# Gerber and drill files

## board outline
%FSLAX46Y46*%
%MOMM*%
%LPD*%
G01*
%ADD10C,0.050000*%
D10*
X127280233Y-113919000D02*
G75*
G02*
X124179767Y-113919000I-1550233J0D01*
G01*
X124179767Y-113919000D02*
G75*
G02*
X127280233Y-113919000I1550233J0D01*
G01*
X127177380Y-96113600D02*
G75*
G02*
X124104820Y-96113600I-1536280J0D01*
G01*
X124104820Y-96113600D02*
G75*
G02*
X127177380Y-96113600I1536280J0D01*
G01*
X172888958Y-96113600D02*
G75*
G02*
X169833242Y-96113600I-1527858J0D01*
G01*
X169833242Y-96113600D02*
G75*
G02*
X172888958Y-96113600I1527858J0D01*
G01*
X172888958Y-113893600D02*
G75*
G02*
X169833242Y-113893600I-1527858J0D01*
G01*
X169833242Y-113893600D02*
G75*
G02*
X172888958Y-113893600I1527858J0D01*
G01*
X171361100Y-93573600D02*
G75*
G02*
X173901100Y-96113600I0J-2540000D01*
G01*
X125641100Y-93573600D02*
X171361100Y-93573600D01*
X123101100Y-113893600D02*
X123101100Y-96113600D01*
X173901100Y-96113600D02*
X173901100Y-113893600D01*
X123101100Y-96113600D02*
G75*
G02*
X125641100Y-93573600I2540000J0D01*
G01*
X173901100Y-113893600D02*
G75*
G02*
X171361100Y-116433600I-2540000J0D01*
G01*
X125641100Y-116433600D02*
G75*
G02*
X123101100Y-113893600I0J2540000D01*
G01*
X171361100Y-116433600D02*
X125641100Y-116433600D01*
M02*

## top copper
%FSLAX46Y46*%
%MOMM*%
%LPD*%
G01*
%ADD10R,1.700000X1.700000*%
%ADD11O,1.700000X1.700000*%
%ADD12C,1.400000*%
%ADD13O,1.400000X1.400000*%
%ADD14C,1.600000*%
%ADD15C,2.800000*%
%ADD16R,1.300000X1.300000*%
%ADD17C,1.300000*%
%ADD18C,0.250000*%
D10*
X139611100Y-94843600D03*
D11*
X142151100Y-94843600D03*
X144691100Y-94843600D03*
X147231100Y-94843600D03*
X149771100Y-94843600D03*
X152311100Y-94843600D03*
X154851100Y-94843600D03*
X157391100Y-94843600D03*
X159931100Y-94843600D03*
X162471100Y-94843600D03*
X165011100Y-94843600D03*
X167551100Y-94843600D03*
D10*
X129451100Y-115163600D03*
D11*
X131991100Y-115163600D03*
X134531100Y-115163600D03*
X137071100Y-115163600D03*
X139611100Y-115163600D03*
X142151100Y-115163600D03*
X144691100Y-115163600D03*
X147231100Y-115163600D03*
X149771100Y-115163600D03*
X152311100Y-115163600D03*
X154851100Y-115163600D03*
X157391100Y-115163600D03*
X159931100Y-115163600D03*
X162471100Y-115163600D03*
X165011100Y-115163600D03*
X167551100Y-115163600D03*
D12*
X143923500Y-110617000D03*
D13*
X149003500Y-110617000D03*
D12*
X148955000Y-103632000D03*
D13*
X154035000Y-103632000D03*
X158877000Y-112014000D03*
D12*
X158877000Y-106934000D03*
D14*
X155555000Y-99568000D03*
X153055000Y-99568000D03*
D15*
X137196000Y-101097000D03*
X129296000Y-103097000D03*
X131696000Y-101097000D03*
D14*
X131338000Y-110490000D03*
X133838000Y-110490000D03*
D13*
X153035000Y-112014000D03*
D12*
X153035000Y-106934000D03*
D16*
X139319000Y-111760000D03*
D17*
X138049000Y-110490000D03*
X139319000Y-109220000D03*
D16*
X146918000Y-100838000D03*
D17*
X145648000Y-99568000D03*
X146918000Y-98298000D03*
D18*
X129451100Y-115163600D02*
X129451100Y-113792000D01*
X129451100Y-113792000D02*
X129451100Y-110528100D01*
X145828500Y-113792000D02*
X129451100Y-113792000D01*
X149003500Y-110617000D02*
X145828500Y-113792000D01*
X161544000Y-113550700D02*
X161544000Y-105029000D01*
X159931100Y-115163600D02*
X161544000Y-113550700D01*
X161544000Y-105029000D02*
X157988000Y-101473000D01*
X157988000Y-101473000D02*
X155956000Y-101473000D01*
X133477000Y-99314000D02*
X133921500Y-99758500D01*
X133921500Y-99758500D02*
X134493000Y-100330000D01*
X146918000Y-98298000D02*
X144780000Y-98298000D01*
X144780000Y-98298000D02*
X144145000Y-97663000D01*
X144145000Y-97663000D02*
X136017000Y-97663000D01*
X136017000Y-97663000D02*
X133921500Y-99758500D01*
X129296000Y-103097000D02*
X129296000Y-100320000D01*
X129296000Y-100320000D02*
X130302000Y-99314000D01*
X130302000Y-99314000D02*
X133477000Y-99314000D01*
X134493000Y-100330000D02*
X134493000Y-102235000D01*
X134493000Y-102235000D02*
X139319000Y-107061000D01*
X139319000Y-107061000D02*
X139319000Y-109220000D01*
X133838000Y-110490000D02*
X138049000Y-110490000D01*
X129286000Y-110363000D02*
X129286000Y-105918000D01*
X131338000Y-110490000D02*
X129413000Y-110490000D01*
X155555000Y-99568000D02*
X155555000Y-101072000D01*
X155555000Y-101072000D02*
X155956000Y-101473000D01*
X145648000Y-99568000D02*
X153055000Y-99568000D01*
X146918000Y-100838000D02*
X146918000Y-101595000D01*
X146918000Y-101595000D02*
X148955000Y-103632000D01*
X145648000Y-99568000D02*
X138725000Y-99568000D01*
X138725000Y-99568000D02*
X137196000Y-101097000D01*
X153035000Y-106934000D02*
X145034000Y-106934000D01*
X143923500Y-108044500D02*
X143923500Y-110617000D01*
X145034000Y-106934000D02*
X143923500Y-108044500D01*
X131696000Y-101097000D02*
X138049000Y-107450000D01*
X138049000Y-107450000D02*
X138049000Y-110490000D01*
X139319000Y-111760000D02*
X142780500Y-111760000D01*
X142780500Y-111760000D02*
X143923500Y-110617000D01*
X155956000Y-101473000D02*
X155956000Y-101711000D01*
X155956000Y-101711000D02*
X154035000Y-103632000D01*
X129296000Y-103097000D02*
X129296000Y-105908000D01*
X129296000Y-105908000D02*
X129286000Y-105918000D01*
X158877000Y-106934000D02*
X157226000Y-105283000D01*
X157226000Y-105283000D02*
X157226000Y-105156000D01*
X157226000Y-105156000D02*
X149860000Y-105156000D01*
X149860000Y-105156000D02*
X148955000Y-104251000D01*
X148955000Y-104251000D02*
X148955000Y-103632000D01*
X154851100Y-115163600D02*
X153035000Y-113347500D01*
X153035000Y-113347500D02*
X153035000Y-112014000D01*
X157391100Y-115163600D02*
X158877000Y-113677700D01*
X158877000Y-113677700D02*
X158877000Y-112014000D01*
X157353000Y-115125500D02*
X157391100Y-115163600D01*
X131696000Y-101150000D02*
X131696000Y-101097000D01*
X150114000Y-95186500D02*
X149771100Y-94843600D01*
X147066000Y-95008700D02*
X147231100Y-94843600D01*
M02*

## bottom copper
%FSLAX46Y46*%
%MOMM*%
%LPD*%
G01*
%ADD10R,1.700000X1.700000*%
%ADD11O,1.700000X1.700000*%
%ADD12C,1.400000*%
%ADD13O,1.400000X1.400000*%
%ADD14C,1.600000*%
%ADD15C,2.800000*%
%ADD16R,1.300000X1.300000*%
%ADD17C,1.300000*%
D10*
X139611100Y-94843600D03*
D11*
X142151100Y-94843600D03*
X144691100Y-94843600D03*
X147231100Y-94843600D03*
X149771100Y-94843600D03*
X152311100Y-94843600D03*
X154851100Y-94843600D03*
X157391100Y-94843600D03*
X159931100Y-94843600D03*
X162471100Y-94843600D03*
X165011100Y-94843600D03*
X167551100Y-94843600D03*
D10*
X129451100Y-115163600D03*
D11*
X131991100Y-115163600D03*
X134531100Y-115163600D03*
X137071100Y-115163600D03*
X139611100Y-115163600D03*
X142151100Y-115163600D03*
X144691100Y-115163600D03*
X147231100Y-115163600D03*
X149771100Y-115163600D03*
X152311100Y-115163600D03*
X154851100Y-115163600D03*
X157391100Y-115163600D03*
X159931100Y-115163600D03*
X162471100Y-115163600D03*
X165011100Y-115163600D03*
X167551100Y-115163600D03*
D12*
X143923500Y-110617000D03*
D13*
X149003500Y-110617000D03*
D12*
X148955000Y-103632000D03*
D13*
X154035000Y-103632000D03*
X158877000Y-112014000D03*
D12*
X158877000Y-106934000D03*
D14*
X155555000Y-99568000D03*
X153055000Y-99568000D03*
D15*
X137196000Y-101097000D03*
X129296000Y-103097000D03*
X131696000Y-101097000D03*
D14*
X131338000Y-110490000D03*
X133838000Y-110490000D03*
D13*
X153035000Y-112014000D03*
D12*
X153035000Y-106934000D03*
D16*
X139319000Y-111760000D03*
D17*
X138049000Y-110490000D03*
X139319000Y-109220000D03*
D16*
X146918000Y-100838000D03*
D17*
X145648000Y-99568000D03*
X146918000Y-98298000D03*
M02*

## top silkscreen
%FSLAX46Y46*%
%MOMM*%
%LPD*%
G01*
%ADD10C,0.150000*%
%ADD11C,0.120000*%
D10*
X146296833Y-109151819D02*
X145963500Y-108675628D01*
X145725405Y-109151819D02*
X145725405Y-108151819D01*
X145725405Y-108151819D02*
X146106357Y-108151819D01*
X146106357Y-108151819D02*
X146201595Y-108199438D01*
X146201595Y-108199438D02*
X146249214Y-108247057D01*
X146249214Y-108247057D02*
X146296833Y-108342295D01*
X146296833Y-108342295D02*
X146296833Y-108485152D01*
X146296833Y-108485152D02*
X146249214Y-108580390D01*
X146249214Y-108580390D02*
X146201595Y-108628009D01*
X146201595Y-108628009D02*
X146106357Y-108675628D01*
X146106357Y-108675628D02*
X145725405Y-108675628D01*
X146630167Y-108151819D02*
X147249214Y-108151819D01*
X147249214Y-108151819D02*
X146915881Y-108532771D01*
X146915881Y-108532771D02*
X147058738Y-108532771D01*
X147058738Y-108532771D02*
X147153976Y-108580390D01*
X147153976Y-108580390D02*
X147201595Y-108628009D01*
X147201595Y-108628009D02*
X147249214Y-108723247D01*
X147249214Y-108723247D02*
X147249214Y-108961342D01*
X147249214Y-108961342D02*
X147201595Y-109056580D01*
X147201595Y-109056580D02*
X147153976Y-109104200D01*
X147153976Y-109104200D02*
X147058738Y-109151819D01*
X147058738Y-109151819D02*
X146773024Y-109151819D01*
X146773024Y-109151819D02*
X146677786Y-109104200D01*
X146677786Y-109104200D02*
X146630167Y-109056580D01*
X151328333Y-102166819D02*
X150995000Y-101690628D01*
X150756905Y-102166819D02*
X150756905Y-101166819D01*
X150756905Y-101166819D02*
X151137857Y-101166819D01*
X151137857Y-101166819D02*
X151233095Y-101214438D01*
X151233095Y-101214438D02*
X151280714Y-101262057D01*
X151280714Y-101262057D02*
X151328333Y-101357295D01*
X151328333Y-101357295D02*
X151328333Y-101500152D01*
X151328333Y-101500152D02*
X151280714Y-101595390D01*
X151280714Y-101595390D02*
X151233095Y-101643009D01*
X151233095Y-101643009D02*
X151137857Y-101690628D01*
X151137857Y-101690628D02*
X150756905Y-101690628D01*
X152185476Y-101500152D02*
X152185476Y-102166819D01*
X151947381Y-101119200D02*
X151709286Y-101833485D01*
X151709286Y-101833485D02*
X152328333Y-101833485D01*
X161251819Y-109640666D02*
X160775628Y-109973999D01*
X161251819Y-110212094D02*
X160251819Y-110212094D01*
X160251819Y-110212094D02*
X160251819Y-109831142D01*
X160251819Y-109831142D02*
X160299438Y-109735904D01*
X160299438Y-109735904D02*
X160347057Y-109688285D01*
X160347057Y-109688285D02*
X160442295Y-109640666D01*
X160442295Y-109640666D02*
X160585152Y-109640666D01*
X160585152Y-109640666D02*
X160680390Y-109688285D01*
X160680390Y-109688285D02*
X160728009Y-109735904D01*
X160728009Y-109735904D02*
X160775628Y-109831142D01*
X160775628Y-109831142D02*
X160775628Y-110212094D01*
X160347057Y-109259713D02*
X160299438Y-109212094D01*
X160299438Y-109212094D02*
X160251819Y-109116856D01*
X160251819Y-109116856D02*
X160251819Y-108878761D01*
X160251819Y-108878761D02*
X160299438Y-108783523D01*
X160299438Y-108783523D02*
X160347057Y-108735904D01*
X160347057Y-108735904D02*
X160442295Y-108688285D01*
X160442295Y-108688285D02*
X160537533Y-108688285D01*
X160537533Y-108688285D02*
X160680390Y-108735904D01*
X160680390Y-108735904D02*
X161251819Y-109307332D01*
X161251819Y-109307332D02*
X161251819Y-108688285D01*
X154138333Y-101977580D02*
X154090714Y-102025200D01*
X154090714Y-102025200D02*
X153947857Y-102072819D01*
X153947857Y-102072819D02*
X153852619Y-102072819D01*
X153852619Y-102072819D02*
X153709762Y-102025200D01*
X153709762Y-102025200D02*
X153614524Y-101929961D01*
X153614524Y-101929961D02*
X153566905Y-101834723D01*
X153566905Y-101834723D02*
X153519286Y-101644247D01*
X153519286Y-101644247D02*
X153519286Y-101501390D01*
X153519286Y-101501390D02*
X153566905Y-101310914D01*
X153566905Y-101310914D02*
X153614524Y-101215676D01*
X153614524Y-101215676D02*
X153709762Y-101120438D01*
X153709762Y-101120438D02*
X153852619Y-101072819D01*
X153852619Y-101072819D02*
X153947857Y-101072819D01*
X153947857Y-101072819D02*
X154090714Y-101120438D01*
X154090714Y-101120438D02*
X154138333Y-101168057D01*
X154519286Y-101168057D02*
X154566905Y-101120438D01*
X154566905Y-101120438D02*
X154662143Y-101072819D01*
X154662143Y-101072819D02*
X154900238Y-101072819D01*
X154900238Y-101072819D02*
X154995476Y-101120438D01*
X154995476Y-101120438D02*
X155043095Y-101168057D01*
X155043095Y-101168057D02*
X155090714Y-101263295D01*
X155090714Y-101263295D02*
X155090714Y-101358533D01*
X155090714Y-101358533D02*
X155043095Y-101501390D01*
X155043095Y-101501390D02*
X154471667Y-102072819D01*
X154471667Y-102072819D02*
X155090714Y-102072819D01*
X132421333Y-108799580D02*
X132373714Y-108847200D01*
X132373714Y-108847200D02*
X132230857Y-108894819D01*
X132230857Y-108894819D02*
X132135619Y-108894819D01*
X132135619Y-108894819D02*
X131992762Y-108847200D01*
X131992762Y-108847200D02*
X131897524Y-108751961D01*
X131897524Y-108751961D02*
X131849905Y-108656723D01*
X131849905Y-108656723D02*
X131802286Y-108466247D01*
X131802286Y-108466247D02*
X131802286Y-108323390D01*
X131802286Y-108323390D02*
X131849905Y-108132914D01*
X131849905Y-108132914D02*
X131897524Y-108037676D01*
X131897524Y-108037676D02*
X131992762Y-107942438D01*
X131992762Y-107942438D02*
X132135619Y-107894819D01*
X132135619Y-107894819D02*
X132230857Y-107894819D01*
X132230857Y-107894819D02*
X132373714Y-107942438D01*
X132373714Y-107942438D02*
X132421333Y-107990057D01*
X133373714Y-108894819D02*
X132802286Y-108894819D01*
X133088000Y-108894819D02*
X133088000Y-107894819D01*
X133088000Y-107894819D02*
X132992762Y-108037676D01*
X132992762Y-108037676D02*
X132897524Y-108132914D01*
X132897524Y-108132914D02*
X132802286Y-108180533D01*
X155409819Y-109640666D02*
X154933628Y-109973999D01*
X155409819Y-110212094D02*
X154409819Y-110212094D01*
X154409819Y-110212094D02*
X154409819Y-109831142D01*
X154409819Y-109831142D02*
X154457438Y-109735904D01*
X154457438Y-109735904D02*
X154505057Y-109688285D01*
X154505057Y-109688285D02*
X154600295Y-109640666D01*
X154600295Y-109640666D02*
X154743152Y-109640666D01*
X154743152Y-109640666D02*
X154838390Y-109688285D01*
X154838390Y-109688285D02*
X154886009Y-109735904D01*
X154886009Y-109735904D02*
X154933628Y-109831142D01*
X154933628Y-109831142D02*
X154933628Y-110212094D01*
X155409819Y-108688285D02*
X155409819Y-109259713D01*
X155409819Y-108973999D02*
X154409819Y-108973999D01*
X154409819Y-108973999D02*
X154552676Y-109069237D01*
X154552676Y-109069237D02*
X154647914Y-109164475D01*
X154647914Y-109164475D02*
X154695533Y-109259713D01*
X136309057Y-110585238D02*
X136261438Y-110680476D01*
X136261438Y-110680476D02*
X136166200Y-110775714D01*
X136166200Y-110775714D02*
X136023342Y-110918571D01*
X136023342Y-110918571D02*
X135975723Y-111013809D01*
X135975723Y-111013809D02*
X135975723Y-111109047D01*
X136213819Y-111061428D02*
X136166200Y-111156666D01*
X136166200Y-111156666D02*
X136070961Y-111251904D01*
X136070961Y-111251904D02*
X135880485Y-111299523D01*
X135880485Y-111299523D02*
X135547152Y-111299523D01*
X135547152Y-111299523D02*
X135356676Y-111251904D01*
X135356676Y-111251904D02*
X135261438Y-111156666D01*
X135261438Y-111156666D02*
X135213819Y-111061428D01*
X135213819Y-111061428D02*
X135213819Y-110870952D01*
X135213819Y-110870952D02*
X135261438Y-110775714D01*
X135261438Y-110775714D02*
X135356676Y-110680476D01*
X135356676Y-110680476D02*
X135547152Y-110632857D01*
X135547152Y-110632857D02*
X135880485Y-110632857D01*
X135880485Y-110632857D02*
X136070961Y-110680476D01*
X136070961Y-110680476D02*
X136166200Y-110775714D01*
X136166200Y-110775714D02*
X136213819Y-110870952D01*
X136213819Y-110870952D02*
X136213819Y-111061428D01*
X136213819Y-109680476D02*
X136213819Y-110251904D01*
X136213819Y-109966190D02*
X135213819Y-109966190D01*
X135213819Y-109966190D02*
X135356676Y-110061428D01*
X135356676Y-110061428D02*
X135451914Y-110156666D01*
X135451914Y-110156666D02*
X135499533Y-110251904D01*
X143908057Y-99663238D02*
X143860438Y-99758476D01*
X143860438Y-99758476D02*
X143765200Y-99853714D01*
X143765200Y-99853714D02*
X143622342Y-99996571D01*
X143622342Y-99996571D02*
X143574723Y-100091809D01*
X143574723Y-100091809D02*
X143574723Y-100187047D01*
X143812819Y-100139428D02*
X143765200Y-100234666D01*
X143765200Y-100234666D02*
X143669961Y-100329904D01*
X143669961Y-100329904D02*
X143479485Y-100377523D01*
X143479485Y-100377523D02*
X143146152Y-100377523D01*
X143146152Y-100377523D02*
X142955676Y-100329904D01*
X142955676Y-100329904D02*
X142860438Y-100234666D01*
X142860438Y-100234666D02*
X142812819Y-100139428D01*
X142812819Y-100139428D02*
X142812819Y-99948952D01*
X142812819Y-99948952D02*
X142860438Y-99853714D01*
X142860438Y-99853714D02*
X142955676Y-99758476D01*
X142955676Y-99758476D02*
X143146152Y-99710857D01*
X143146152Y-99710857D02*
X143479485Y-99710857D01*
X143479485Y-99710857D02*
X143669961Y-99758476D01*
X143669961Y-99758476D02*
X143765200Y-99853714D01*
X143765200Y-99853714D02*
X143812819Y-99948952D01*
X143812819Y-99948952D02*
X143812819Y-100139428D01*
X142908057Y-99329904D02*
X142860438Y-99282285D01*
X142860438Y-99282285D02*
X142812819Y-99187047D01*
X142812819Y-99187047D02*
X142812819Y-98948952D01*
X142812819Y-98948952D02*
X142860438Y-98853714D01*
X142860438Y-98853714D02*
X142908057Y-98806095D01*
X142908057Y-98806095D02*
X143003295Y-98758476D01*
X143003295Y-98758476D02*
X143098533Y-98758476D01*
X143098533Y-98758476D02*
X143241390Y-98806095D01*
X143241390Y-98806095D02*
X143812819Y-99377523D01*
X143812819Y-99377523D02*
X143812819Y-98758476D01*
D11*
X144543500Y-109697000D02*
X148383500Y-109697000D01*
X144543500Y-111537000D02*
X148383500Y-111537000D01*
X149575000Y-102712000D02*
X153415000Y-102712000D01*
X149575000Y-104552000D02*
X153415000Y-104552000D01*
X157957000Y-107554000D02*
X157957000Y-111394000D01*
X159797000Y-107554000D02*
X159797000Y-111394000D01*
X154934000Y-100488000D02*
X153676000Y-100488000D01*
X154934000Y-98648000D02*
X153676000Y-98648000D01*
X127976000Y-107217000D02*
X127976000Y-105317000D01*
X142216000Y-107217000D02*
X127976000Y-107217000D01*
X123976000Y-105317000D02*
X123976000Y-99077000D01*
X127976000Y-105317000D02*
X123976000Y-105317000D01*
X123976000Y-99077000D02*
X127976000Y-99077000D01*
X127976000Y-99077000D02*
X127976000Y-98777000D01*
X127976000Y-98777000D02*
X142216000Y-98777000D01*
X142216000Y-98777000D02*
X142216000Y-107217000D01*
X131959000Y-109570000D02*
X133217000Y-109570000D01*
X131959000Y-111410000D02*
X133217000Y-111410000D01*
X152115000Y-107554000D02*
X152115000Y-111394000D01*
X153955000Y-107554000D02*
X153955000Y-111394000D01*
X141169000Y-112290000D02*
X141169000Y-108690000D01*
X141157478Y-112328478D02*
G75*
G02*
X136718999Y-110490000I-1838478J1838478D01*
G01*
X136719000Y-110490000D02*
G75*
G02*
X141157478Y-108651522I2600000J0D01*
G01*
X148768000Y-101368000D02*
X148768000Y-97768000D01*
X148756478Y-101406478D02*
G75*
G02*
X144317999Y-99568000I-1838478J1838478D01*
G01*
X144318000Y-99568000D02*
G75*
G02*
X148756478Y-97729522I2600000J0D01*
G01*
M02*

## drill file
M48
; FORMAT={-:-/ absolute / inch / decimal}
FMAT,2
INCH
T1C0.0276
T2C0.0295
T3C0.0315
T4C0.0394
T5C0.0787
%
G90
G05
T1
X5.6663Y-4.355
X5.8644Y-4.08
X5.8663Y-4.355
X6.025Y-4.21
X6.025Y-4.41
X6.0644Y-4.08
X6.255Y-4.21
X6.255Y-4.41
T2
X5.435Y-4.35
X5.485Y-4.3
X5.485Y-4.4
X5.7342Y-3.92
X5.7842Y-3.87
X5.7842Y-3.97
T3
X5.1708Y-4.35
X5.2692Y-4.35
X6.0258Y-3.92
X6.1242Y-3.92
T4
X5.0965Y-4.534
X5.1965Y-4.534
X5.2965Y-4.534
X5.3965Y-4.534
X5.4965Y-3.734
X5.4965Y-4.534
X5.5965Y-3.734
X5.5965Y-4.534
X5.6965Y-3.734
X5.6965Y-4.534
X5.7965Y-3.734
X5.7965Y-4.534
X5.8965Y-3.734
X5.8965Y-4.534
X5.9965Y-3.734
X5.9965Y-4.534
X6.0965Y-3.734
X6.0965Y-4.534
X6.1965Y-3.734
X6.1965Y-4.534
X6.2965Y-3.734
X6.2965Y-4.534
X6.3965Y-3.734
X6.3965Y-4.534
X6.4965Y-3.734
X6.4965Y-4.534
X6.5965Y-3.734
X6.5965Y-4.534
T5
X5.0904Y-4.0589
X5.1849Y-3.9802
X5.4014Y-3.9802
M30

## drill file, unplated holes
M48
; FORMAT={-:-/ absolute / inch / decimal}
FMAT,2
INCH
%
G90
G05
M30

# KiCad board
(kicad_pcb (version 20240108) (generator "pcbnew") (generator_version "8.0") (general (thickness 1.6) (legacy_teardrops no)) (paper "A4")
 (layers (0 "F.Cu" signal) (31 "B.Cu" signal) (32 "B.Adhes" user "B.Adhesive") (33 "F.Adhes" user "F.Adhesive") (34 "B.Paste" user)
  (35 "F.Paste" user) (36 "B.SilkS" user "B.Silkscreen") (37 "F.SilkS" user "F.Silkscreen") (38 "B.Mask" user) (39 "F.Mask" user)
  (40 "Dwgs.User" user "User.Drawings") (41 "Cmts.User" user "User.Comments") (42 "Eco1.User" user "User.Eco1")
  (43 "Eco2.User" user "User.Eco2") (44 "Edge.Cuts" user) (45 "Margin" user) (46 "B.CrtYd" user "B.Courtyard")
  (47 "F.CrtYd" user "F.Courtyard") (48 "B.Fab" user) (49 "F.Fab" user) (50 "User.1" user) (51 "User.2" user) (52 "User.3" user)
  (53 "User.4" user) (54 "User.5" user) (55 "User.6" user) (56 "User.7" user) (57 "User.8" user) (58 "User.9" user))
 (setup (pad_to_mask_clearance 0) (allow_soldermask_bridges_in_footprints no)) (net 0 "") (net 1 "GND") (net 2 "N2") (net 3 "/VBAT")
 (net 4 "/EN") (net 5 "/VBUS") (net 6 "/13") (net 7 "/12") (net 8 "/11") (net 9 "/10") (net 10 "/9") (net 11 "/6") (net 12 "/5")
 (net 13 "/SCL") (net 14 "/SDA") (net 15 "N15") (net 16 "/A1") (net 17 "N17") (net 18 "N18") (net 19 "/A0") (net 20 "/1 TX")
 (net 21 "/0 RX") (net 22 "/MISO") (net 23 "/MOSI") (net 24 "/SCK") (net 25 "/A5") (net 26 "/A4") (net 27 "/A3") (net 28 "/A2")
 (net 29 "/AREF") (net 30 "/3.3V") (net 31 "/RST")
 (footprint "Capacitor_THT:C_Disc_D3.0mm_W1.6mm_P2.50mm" (layer "F.Cu") (at 155.555 99.568 180)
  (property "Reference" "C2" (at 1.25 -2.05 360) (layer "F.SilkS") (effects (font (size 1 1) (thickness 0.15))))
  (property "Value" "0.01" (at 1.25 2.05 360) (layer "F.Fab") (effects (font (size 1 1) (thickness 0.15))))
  (fp_line (start 0.621 0.92) (end 1.879 0.92) (stroke (width 0.12) (type solid)) (layer "F.SilkS"))
  (fp_line (start 0.621 -0.92) (end 1.879 -0.92) (stroke (width 0.12) (type solid)) (layer "F.SilkS"))
  (pad "1" thru_hole circle (at 0 0 180) (size 1.6 1.6) (drill 0.8) (layers "*.Cu" "*.Mask") (remove_unused_layers no) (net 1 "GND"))
  (pad "2" thru_hole circle (at 2.5 0 180) (size 1.6 1.6) (drill 0.8) (layers "*.Cu" "*.Mask") (remove_unused_layers no) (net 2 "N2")))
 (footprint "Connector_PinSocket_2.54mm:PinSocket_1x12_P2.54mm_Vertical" (layer "F.Cu") (at 139.6111 94.8436 90)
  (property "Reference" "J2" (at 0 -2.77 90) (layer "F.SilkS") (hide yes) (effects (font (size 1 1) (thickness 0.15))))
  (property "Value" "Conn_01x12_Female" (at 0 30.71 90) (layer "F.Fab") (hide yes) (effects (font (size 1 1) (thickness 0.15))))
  (pad "1" thru_hole rect (at 0 0 90) (size 1.7 1.7) (drill 1) (layers "*.Cu" "*.Mask") (remove_unused_layers no) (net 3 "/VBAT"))
  (pad "2" thru_hole oval (at 0 2.54 90) (size 1.7 1.7) (drill 1) (layers "*.Cu" "*.Mask") (remove_unused_layers no) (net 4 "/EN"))
  (pad "3" thru_hole oval (at 0 5.08 90) (size 1.7 1.7) (drill 1) (layers "*.Cu" "*.Mask") (remove_unused_layers no) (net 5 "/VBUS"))
  (pad "4" thru_hole oval (at 0 7.62 90) (size 1.7 1.7) (drill 1) (layers "*.Cu" "*.Mask") (remove_unused_layers no) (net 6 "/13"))
  (pad "5" thru_hole oval (at 0 10.16 90) (size 1.7 1.7) (drill 1) (layers "*.Cu" "*.Mask") (remove_unused_layers no) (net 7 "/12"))
  (pad "6" thru_hole oval (at 0 12.7 90) (size 1.7 1.7) (drill 1) (layers "*.Cu" "*.Mask") (remove_unused_layers no) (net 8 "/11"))
  (pad "7" thru_hole oval (at 0 15.24 90) (size 1.7 1.7) (drill 1) (layers "*.Cu" "*.Mask") (remove_unused_layers no) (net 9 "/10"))
  (pad "8" thru_hole oval (at 0 17.78 90) (size 1.7 1.7) (drill 1) (layers "*.Cu" "*.Mask") (remove_unused_layers no) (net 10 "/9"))
  (pad "9" thru_hole oval (at 0 20.32 90) (size 1.7 1.7) (drill 1) (layers "*.Cu" "*.Mask") (remove_unused_layers no) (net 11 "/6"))
  (pad "10" thru_hole oval (at 0 22.86 90) (size 1.7 1.7) (drill 1) (layers "*.Cu" "*.Mask") (remove_unused_layers no) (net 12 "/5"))
  (pad "11" thru_hole oval (at 0 25.4 90) (size 1.7 1.7) (drill 1) (layers "*.Cu" "*.Mask") (remove_unused_layers no) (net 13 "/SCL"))
  (pad "12" thru_hole oval (at 0 27.94 90) (size 1.7 1.7) (drill 1) (layers "*.Cu" "*.Mask") (remove_unused_layers no) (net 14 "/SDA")))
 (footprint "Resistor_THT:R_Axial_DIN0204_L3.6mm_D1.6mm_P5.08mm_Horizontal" (layer "F.Cu") (at 153.035 106.934 -90)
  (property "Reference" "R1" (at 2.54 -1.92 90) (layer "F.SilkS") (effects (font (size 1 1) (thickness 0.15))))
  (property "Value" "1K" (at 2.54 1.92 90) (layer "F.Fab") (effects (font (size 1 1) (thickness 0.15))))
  (fp_line (start 0.62 0.92) (end 4.46 0.92) (stroke (width 0.12) (type solid)) (layer "F.SilkS"))
  (fp_line (start 0.62 -0.92) (end 4.46 -0.92) (stroke (width 0.12) (type solid)) (layer "F.SilkS"))
  (pad "1" thru_hole circle (at 0 0 270) (size 1.4 1.4) (drill 0.7) (layers "*.Cu" "*.Mask") (remove_unused_layers no) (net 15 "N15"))
  (pad "2" thru_hole oval (at 5.08 0 270) (size 1.4 1.4) (drill 0.7) (layers "*.Cu" "*.Mask") (remove_unused_layers no) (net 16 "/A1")))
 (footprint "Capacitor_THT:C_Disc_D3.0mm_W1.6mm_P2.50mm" (layer "F.Cu") (at 131.338 110.49)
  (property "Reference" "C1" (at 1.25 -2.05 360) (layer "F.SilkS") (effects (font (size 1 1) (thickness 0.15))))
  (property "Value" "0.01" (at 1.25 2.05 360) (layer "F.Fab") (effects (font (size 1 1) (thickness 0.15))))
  (fp_line (start 0.621 -0.92) (end 1.879 -0.92) (stroke (width 0.12) (type solid)) (layer "F.SilkS"))
  (fp_line (start 0.621 0.92) (end 1.879 0.92) (stroke (width 0.12) (type solid)) (layer "F.SilkS"))
  (pad "1" thru_hole circle (at 0 0) (size 1.6 1.6) (drill 0.8) (layers "*.Cu" "*.Mask") (remove_unused_layers no) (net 1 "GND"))
  (pad "2" thru_hole circle (at 2.5 0) (size 1.6 1.6) (drill 0.8) (layers "*.Cu" "*.Mask") (remove_unused_layers no) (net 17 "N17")))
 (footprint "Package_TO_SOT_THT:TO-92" (layer "F.Cu") (at 146.918 100.838 90)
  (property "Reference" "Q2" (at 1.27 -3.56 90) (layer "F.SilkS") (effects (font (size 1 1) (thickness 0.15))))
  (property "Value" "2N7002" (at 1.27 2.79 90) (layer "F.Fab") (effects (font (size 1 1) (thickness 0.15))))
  (fp_line (start -0.53 1.85) (end 3.07 1.85) (stroke (width 0.12) (type solid)) (layer "F.SilkS"))
  (fp_arc (start 1.27 -2.6) (mid 3.672087 -0.994977) (end 3.108478 1.838478) (stroke (width 0.12) (type solid)) (layer "F.SilkS"))
  (fp_arc (start -0.568478 1.838478) (mid -1.132087 -0.994977) (end 1.27 -2.6) (stroke (width 0.12) (type solid)) (layer "F.SilkS"))
  (pad "1" thru_hole rect (at 0 0 90) (size 1.3 1.3) (drill 0.75) (layers "*.Cu" "*.Mask") (remove_unused_layers no) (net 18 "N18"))
  (pad "2" thru_hole circle (at 1.27 -1.27 90) (size 1.3 1.3) (drill 0.75) (layers "*.Cu" "*.Mask") (remove_unused_layers no) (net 2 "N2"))
  (pad "3" thru_hole circle (at 2.54 0 90) (size 1.3 1.3) (drill 0.75) (layers "*.Cu" "*.Mask") (remove_unused_layers no) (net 1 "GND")))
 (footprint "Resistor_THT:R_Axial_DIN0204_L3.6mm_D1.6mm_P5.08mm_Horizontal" (layer "F.Cu") (at 158.877 106.934 -90)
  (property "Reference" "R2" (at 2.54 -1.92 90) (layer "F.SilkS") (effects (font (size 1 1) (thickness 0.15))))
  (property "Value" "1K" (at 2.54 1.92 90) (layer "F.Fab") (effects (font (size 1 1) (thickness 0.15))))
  (fp_line (start 0.62 0.92) (end 4.46 0.92) (stroke (width 0.12) (type solid)) (layer "F.SilkS"))
  (fp_line (start 0.62 -0.92) (end 4.46 -0.92) (stroke (width 0.12) (type solid)) (layer "F.SilkS"))
  (pad "1" thru_hole circle (at 0 0 270) (size 1.4 1.4) (drill 0.7) (layers "*.Cu" "*.Mask") (remove_unused_layers no) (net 18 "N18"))
  (pad "2" thru_hole oval (at 5.08 0 270) (size 1.4 1.4) (drill 0.7) (layers "*.Cu" "*.Mask") (remove_unused_layers no) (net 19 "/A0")))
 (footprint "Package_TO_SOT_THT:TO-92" (layer "F.Cu") (at 139.319 111.76 90)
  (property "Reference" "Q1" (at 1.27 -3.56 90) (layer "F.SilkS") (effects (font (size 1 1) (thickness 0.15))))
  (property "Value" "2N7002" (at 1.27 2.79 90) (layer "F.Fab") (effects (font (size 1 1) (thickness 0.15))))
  (fp_line (start -0.53 1.85) (end 3.07 1.85) (stroke (width 0.12) (type solid)) (layer "F.SilkS"))
  (fp_arc (start 1.27 -2.6) (mid 3.672087 -0.994977) (end 3.108478 1.838478) (stroke (width 0.12) (type solid)) (layer "F.SilkS"))
  (fp_arc (start -0.568478 1.838478) (mid -1.132087 -0.994977) (end 1.27 -2.6) (stroke (width 0.12) (type solid)) (layer "F.SilkS"))
  (pad "1" thru_hole rect (at 0 0 90) (size 1.3 1.3) (drill 0.75) (layers "*.Cu" "*.Mask") (remove_unused_layers no) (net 15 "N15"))
  (pad "2" thru_hole circle (at 1.27 -1.27 90) (size 1.3 1.3) (drill 0.75) (layers "*.Cu" "*.Mask") (remove_unused_layers no) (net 17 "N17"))
  (pad "3" thru_hole circle (at 2.54 0 90) (size 1.3 1.3) (drill 0.75) (layers "*.Cu" "*.Mask") (remove_unused_layers no) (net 1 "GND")))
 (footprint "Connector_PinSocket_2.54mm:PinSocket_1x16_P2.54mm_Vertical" (layer "F.Cu") (at 129.4511 115.1636 90)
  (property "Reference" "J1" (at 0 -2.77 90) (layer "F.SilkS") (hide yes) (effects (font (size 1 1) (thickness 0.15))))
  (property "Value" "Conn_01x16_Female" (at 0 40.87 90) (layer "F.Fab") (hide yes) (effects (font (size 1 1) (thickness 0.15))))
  (pad "1" thru_hole rect (at 0 0 90) (size 1.7 1.7) (drill 1) (layers "*.Cu" "*.Mask") (remove_unused_layers no) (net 1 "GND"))
  (pad "2" thru_hole oval (at 0 2.54 90) (size 1.7 1.7) (drill 1) (layers "*.Cu" "*.Mask") (remove_unused_layers no) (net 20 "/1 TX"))
  (pad "3" thru_hole oval (at 0 5.08 90) (size 1.7 1.7) (drill 1) (layers "*.Cu" "*.Mask") (remove_unused_layers no) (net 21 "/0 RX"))
  (pad "4" thru_hole oval (at 0 7.62 90) (size 1.7 1.7) (drill 1) (layers "*.Cu" "*.Mask") (remove_unused_layers no) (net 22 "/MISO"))
  (pad "5" thru_hole oval (at 0 10.16 90) (size 1.7 1.7) (drill 1) (layers "*.Cu" "*.Mask") (remove_unused_layers no) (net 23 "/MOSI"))
  (pad "6" thru_hole oval (at 0 12.7 90) (size 1.7 1.7) (drill 1) (layers "*.Cu" "*.Mask") (remove_unused_layers no) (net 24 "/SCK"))
  (pad "7" thru_hole oval (at 0 15.24 90) (size 1.7 1.7) (drill 1) (layers "*.Cu" "*.Mask") (remove_unused_layers no) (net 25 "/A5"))
  (pad "8" thru_hole oval (at 0 17.78 90) (size 1.7 1.7) (drill 1) (layers "*.Cu" "*.Mask") (remove_unused_layers no) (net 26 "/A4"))
  (pad "9" thru_hole oval (at 0 20.32 90) (size 1.7 1.7) (drill 1) (layers "*.Cu" "*.Mask") (remove_unused_layers no) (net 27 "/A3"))
  (pad "10" thru_hole oval (at 0 22.86 90) (size 1.7 1.7) (drill 1) (layers "*.Cu" "*.Mask") (remove_unused_layers no) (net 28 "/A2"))
  (pad "11" thru_hole oval (at 0 25.4 90) (size 1.7 1.7) (drill 1) (layers "*.Cu" "*.Mask") (remove_unused_layers no) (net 16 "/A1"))
  (pad "12" thru_hole oval (at 0 27.94 90) (size 1.7 1.7) (drill 1) (layers "*.Cu" "*.Mask") (remove_unused_layers no) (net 19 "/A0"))
  (pad "13" thru_hole oval (at 0 30.48 90) (size 1.7 1.7) (drill 1) (layers "*.Cu" "*.Mask") (remove_unused_layers no) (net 1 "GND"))
  (pad "14" thru_hole oval (at 0 33.02 90) (size 1.7 1.7) (drill 1) (layers "*.Cu" "*.Mask") (remove_unused_layers no) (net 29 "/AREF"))
  (pad "15" thru_hole oval (at 0 35.56 90) (size 1.7 1.7) (drill 1) (layers "*.Cu" "*.Mask") (remove_unused_layers no) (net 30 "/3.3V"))
  (pad "16" thru_hole oval (at 0 38.1 90) (size 1.7 1.7) (drill 1) (layers "*.Cu" "*.Mask") (remove_unused_layers no) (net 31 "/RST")))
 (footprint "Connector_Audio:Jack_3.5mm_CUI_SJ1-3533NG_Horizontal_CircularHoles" (layer "F.Cu") (at 129.296 103.097 90)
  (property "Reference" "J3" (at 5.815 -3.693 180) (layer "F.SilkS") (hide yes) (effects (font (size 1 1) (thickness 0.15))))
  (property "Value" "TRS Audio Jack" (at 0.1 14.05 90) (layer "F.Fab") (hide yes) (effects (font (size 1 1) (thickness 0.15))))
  (fp_line (start 4.02 -5.32) (end 4.02 -1.32) (stroke (width 0.12) (type solid)) (layer "F.SilkS"))
  (fp_line (start -2.22 -5.32) (end 4.02 -5.32) (stroke (width 0.12) (type solid)) (layer "F.SilkS"))
  (fp_line (start 4.32 -1.32) (end 4.32 12.92) (stroke (width 0.12) (type solid)) (layer "F.SilkS"))
  (fp_line (start 4.02 -1.32) (end 4.32 -1.32) (stroke (width 0.12) (type solid)) (layer "F.SilkS"))
  (fp_line (start -2.22 -1.32) (end -2.22 -5.32) (stroke (width 0.12) (type solid)) (layer "F.SilkS"))
  (fp_line (start -4.12 -1.32) (end -2.22 -1.32) (stroke (width 0.12) (type solid)) (layer "F.SilkS"))
  (fp_line (start 4.32 12.92) (end -4.12 12.92) (stroke (width 0.12) (type solid)) (layer "F.SilkS"))
  (fp_line (start -4.12 12.92) (end -4.12 -1.32) (stroke (width 0.12) (type solid)) (layer "F.SilkS"))
  (pad "R" thru_hole circle (at 2 7.9 90) (size 2.8 2.8) (drill 2) (layers "*.Cu" "*.Mask") (remove_unused_layers no) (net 2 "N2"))
  (pad "S" thru_hole circle (at 0 0 90) (size 2.8 2.8) (drill 2) (layers "*.Cu" "*.Mask") (remove_unused_layers no) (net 1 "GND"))
  (pad "T" thru_hole circle (at 2 2.4 90) (size 2.8 2.8) (drill 2) (layers "*.Cu" "*.Mask") (remove_unused_layers no) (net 17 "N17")))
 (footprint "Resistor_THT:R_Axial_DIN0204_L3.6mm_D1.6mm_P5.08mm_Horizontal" (layer "F.Cu") (at 143.9235 110.617)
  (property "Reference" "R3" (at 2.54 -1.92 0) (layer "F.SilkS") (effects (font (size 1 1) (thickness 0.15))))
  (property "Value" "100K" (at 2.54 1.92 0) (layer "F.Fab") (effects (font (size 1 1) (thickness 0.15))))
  (fp_line (start 0.62 -0.92) (end 4.46 -0.92) (stroke (width 0.12) (type solid)) (layer "F.SilkS"))
  (fp_line (start 0.62 0.92) (end 4.46 0.92) (stroke (width 0.12) (type solid)) (layer "F.SilkS"))
  (pad "1" thru_hole circle (at 0 0) (size 1.4 1.4) (drill 0.7) (layers "*.Cu" "*.Mask") (remove_unused_layers no) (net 15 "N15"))
  (pad "2" thru_hole oval (at 5.08 0) (size 1.4 1.4) (drill 0.7) (layers "*.Cu" "*.Mask") (remove_unused_layers no) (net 1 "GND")))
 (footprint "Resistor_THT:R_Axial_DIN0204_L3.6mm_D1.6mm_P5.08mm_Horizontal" (layer "F.Cu") (at 148.955 103.632)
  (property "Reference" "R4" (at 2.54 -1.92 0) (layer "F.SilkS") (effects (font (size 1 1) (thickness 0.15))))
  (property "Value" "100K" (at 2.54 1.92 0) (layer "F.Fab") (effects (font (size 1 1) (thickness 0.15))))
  (fp_line (start 0.62 -0.92) (end 4.46 -0.92) (stroke (width 0.12) (type solid)) (layer "F.SilkS"))
  (fp_line (start 0.62 0.92) (end 4.46 0.92) (stroke (width 0.12) (type solid)) (layer "F.SilkS"))
  (pad "1" thru_hole circle (at 0 0) (size 1.4 1.4) (drill 0.7) (layers "*.Cu" "*.Mask") (remove_unused_layers no) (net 18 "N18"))
  (pad "2" thru_hole oval (at 5.08 0) (size 1.4 1.4) (drill 0.7) (layers "*.Cu" "*.Mask") (remove_unused_layers no) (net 1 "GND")))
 (gr_circle (center 171.3611 113.8936) (end 170.688 112.522) (stroke (width 0.05) (type default)) (fill none) (layer "Edge.Cuts"))
 (gr_circle (center 125.73 113.919) (end 124.841 112.649) (stroke (width 0.05) (type default)) (fill none) (layer "Edge.Cuts"))
 (gr_arc (start 171.3611 93.5736) (mid 173.157151 94.317549) (end 173.9011 96.1136) (stroke (width 0.05) (type solid)) (layer "Edge.Cuts"))
 (gr_line (start 125.6411 93.5736) (end 171.3611 93.5736) (stroke (width 0.05) (type solid)) (layer "Edge.Cuts"))
 (gr_line (start 123.1011 113.8936) (end 123.1011 96.1136) (stroke (width 0.05) (type solid)) (layer "Edge.Cuts"))
 (gr_line (start 173.9011 96.1136) (end 173.9011 113.8936) (stroke (width 0.05) (type solid)) (layer "Edge.Cuts"))
 (gr_arc (start 123.1011 96.1136) (mid 123.845049 94.317549) (end 125.6411 93.5736) (stroke (width 0.05) (type solid)) (layer "Edge.Cuts"))
 (gr_arc (start 173.9011 113.8936) (mid 173.157151 115.689651) (end 171.3611 116.4336) (stroke (width 0.05) (type solid))
  (layer "Edge.Cuts"))
 (gr_arc (start 125.6411 116.4336) (mid 123.845049 115.689651) (end 123.1011 113.8936) (stroke (width 0.05) (type solid))
  (layer "Edge.Cuts"))
 (gr_circle (center 125.6411 96.1136) (end 124.587 94.996) (stroke (width 0.05) (type default)) (fill none) (layer "Edge.Cuts"))
 (gr_line (start 171.3611 116.4336) (end 125.6411 116.4336) (stroke (width 0.05) (type solid)) (layer "Edge.Cuts"))
 (gr_circle (center 171.3611 96.1136) (end 170.688 94.742) (stroke (width 0.05) (type default)) (fill none) (layer "Edge.Cuts"))
 (segment (start 134.493 100.33) (end 134.493 102.235) (width 0.25) (layer "F.Cu") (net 1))
 (segment (start 149.0035 110.617) (end 145.8285 113.792) (width 0.25) (layer "F.Cu") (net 1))
 (segment (start 136.017 97.663) (end 133.9215 99.7585) (width 0.25) (layer "F.Cu") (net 1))
 (segment (start 161.544 113.5507) (end 161.544 105.029) (width 0.25) (layer "F.Cu") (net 1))
 (segment (start 129.4511 113.792) (end 129.4511 110.5281) (width 0.25) (layer "F.Cu") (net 1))
 (segment (start 129.296 105.908) (end 129.286 105.918) (width 0.25) (layer "F.Cu") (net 1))
 (segment (start 161.544 105.029) (end 157.988 101.473) (width 0.25) (layer "F.Cu") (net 1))
 (segment (start 129.296 103.097) (end 129.296 100.32) (width 0.25) (layer "F.Cu") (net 1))
 (segment (start 129.4511 115.1636) (end 129.4511 113.792) (width 0.25) (layer "F.Cu") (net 1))
 (segment (start 133.9215 99.7585) (end 134.493 100.33) (width 0.25) (layer "F.Cu") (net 1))
 (segment (start 133.477 99.314) (end 133.9215 99.7585) (width 0.25) (layer "F.Cu") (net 1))
 (segment (start 131.338 110.49) (end 129.413 110.49) (width 0.25) (layer "F.Cu") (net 1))
 (segment (start 155.555 101.072) (end 155.956 101.473) (width 0.25) (layer "F.Cu") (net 1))
 (segment (start 144.78 98.298) (end 144.145 97.663) (width 0.25) (layer "F.Cu") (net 1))
 (segment (start 145.8285 113.792) (end 129.4511 113.792) (width 0.25) (layer "F.Cu") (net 1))
 (segment (start 134.493 102.235) (end 139.319 107.061) (width 0.25) (layer "F.Cu") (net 1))
 (segment (start 155.956 101.711) (end 154.035 103.632) (width 0.25) (layer "F.Cu") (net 1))
 (segment (start 129.286 110.363) (end 129.286 105.918) (width 0.25) (layer "F.Cu") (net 1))
 (segment (start 157.988 101.473) (end 155.956 101.473) (width 0.25) (layer "F.Cu") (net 1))
 (segment (start 146.918 98.298) (end 144.78 98.298) (width 0.25) (layer "F.Cu") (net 1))
 (segment (start 139.319 107.061) (end 139.319 109.22) (width 0.25) (layer "F.Cu") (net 1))
 (segment (start 130.302 99.314) (end 133.477 99.314) (width 0.25) (layer "F.Cu") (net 1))
 (segment (start 155.956 101.473) (end 155.956 101.711) (width 0.25) (layer "F.Cu") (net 1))
 (segment (start 155.555 99.568) (end 155.555 101.072) (width 0.25) (layer "F.Cu") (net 1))
 (segment (start 129.296 100.32) (end 130.302 99.314) (width 0.25) (layer "F.Cu") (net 1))
 (segment (start 129.296 103.097) (end 129.296 105.908) (width 0.25) (layer "F.Cu") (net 1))
 (segment (start 159.9311 115.1636) (end 161.544 113.5507) (width 0.25) (layer "F.Cu") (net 1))
 (segment (start 144.145 97.663) (end 136.017 97.663) (width 0.25) (layer "F.Cu") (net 1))
 (segment (start 153.035 113.3475) (end 153.035 112.014) (width 0.25) (layer "F.Cu") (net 16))
 (segment (start 154.8511 115.1636) (end 153.035 113.3475) (width 0.25) (layer "F.Cu") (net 16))
 (segment (start 158.877 113.6777) (end 158.877 112.014) (width 0.25) (layer "F.Cu") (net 19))
 (segment (start 157.353 115.1255) (end 157.3911 115.1636) (width 0.25) (layer "F.Cu") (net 19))
 (segment (start 157.3911 115.1636) (end 158.877 113.6777) (width 0.25) (layer "F.Cu") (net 19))
 (segment (start 147.066 95.0087) (end 147.2311 94.8436) (width 0.25) (layer "F.Cu") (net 6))
 (segment (start 150.114 95.1865) (end 149.7711 94.8436) (width 0.25) (layer "F.Cu") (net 7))
 (segment (start 139.319 111.76) (end 142.7805 111.76) (width 0.25) (layer "F.Cu") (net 15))
 (segment (start 145.034 106.934) (end 143.9235 108.0445) (width 0.25) (layer "F.Cu") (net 15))
 (segment (start 153.035 106.934) (end 145.034 106.934) (width 0.25) (layer "F.Cu") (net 15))
 (segment (start 143.9235 108.0445) (end 143.9235 110.617) (width 0.25) (layer "F.Cu") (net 15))
 (segment (start 142.7805 111.76) (end 143.9235 110.617) (width 0.25) (layer "F.Cu") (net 15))
 (segment (start 133.838 110.49) (end 138.049 110.49) (width 0.25) (layer "F.Cu") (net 17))
 (segment (start 138.049 107.45) (end 138.049 110.49) (width 0.25) (layer "F.Cu") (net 17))
 (segment (start 131.696 101.15) (end 131.696 101.097) (width 0.25) (layer "F.Cu") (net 17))
 (segment (start 131.696 101.097) (end 138.049 107.45) (width 0.25) (layer "F.Cu") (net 17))
 (segment (start 145.648 99.568) (end 153.055 99.568) (width 0.25) (layer "F.Cu") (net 2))
 (segment (start 138.725 99.568) (end 137.196 101.097) (width 0.25) (layer "F.Cu") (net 2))
 (segment (start 145.648 99.568) (end 138.725 99.568) (width 0.25) (layer "F.Cu") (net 2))
 (segment (start 157.226 105.156) (end 149.86 105.156) (width 0.25) (layer "F.Cu") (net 18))
 (segment (start 146.918 100.838) (end 146.918 101.595) (width 0.25) (layer "F.Cu") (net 18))
 (segment (start 158.877 106.934) (end 157.226 105.283) (width 0.25) (layer "F.Cu") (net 18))
 (segment (start 146.918 101.595) (end 148.955 103.632) (width 0.25) (layer "F.Cu") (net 18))
 (segment (start 149.86 105.156) (end 148.955 104.251) (width 0.25) (layer "F.Cu") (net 18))
 (segment (start 157.226 105.283) (end 157.226 105.156) (width 0.25) (layer "F.Cu") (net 18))
 (segment (start 148.955 104.251) (end 148.955 103.632) (width 0.25) (layer "F.Cu") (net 18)))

